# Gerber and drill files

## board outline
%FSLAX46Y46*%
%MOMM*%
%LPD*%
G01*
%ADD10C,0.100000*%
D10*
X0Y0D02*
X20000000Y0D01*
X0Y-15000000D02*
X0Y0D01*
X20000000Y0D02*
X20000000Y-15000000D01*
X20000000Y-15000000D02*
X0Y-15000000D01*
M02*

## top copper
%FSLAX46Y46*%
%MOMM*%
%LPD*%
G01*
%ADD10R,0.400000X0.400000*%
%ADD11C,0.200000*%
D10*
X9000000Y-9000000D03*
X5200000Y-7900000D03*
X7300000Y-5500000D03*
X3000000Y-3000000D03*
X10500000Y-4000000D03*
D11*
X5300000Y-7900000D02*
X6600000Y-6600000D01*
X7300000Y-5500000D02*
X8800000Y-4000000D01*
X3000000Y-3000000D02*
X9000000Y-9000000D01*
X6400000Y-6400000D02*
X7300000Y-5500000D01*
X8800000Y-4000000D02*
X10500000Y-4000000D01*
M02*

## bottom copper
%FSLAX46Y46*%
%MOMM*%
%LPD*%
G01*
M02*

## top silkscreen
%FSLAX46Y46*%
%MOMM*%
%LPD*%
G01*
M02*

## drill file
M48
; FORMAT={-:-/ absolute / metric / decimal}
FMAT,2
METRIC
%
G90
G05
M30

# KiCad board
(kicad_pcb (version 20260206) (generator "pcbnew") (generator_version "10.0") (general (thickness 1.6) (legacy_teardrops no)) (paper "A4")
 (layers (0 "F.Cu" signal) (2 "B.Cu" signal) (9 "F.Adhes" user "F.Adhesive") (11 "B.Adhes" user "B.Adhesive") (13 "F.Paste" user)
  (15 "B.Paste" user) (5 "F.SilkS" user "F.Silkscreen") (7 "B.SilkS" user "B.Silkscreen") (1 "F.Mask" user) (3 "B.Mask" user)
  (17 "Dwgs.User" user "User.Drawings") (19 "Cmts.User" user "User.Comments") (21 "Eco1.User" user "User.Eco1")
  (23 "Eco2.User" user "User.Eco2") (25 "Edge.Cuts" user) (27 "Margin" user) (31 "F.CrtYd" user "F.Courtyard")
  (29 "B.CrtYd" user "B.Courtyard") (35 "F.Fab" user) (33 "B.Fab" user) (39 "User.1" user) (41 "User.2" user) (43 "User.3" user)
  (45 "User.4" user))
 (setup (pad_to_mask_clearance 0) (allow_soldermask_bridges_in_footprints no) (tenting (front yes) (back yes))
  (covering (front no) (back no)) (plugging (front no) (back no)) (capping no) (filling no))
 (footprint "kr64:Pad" (layer "F.Cu") (at 9 9)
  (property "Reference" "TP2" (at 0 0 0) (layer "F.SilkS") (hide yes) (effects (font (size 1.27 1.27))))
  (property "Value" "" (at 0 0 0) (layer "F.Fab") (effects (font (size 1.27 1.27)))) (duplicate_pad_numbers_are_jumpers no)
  (pad "1" smd rect (at 0 0) (size 0.4 0.4) (layers "F.Cu" "F.Mask" "F.Paste") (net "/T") (thermal_bridge_angle 45)))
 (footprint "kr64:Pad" (layer "F.Cu") (at 5.2 7.9)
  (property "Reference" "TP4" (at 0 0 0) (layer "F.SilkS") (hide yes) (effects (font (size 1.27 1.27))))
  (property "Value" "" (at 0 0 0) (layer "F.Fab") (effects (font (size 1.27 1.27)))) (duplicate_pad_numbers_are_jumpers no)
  (pad "1" smd rect (at 0 0) (size 0.4 0.4) (layers "F.Cu" "F.Mask" "F.Paste") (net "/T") (thermal_bridge_angle 45)))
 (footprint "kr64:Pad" (layer "F.Cu") (at 7.3 5.5)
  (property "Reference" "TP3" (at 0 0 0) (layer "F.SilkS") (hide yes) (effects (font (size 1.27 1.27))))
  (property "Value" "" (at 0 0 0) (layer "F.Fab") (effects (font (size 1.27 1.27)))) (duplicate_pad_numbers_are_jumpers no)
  (pad "1" smd rect (at 0 0) (size 0.4 0.4) (layers "F.Cu" "F.Mask" "F.Paste") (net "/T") (thermal_bridge_angle 45)))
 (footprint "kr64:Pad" (layer "F.Cu") (at 3 3)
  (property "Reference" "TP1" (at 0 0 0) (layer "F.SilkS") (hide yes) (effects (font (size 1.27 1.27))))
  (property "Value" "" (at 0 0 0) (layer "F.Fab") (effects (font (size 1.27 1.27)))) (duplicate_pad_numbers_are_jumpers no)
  (pad "1" smd rect (at 0 0) (size 0.4 0.4) (layers "F.Cu" "F.Mask" "F.Paste") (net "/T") (thermal_bridge_angle 45)))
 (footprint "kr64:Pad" (layer "F.Cu") (at 10.5 4)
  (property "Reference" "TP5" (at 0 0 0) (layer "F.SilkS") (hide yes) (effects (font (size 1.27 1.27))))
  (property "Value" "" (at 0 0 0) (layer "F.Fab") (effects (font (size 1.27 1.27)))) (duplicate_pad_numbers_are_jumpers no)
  (pad "1" smd rect (at 0 0) (size 0.4 0.4) (layers "F.Cu" "F.Mask" "F.Paste") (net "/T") (thermal_bridge_angle 45)))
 (gr_line (start 0 0) (end 20 0) (stroke (width 0.1) (type default)) (layer "Edge.Cuts"))
 (gr_line (start 0 15) (end 0 0) (stroke (width 0.1) (type default)) (layer "Edge.Cuts"))
 (gr_line (start 20 0) (end 20 15) (stroke (width 0.1) (type default)) (layer "Edge.Cuts"))
 (gr_line (start 20 15) (end 0 15) (stroke (width 0.1) (type default)) (layer "Edge.Cuts"))
 (segment (start 5.3 7.9) (end 6.6 6.6) (width 0.2) (layer "F.Cu") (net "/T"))
 (segment (start 7.3 5.5) (end 8.8 4) (width 0.2) (layer "F.Cu") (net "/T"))
 (segment (start 3 3) (end 9 9) (width 0.2) (layer "F.Cu") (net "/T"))
 (segment (start 6.4 6.4) (end 7.3 5.5) (width 0.2) (layer "F.Cu") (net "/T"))
 (segment (start 8.8 4) (end 10.5 4) (width 0.2) (layer "F.Cu") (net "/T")))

